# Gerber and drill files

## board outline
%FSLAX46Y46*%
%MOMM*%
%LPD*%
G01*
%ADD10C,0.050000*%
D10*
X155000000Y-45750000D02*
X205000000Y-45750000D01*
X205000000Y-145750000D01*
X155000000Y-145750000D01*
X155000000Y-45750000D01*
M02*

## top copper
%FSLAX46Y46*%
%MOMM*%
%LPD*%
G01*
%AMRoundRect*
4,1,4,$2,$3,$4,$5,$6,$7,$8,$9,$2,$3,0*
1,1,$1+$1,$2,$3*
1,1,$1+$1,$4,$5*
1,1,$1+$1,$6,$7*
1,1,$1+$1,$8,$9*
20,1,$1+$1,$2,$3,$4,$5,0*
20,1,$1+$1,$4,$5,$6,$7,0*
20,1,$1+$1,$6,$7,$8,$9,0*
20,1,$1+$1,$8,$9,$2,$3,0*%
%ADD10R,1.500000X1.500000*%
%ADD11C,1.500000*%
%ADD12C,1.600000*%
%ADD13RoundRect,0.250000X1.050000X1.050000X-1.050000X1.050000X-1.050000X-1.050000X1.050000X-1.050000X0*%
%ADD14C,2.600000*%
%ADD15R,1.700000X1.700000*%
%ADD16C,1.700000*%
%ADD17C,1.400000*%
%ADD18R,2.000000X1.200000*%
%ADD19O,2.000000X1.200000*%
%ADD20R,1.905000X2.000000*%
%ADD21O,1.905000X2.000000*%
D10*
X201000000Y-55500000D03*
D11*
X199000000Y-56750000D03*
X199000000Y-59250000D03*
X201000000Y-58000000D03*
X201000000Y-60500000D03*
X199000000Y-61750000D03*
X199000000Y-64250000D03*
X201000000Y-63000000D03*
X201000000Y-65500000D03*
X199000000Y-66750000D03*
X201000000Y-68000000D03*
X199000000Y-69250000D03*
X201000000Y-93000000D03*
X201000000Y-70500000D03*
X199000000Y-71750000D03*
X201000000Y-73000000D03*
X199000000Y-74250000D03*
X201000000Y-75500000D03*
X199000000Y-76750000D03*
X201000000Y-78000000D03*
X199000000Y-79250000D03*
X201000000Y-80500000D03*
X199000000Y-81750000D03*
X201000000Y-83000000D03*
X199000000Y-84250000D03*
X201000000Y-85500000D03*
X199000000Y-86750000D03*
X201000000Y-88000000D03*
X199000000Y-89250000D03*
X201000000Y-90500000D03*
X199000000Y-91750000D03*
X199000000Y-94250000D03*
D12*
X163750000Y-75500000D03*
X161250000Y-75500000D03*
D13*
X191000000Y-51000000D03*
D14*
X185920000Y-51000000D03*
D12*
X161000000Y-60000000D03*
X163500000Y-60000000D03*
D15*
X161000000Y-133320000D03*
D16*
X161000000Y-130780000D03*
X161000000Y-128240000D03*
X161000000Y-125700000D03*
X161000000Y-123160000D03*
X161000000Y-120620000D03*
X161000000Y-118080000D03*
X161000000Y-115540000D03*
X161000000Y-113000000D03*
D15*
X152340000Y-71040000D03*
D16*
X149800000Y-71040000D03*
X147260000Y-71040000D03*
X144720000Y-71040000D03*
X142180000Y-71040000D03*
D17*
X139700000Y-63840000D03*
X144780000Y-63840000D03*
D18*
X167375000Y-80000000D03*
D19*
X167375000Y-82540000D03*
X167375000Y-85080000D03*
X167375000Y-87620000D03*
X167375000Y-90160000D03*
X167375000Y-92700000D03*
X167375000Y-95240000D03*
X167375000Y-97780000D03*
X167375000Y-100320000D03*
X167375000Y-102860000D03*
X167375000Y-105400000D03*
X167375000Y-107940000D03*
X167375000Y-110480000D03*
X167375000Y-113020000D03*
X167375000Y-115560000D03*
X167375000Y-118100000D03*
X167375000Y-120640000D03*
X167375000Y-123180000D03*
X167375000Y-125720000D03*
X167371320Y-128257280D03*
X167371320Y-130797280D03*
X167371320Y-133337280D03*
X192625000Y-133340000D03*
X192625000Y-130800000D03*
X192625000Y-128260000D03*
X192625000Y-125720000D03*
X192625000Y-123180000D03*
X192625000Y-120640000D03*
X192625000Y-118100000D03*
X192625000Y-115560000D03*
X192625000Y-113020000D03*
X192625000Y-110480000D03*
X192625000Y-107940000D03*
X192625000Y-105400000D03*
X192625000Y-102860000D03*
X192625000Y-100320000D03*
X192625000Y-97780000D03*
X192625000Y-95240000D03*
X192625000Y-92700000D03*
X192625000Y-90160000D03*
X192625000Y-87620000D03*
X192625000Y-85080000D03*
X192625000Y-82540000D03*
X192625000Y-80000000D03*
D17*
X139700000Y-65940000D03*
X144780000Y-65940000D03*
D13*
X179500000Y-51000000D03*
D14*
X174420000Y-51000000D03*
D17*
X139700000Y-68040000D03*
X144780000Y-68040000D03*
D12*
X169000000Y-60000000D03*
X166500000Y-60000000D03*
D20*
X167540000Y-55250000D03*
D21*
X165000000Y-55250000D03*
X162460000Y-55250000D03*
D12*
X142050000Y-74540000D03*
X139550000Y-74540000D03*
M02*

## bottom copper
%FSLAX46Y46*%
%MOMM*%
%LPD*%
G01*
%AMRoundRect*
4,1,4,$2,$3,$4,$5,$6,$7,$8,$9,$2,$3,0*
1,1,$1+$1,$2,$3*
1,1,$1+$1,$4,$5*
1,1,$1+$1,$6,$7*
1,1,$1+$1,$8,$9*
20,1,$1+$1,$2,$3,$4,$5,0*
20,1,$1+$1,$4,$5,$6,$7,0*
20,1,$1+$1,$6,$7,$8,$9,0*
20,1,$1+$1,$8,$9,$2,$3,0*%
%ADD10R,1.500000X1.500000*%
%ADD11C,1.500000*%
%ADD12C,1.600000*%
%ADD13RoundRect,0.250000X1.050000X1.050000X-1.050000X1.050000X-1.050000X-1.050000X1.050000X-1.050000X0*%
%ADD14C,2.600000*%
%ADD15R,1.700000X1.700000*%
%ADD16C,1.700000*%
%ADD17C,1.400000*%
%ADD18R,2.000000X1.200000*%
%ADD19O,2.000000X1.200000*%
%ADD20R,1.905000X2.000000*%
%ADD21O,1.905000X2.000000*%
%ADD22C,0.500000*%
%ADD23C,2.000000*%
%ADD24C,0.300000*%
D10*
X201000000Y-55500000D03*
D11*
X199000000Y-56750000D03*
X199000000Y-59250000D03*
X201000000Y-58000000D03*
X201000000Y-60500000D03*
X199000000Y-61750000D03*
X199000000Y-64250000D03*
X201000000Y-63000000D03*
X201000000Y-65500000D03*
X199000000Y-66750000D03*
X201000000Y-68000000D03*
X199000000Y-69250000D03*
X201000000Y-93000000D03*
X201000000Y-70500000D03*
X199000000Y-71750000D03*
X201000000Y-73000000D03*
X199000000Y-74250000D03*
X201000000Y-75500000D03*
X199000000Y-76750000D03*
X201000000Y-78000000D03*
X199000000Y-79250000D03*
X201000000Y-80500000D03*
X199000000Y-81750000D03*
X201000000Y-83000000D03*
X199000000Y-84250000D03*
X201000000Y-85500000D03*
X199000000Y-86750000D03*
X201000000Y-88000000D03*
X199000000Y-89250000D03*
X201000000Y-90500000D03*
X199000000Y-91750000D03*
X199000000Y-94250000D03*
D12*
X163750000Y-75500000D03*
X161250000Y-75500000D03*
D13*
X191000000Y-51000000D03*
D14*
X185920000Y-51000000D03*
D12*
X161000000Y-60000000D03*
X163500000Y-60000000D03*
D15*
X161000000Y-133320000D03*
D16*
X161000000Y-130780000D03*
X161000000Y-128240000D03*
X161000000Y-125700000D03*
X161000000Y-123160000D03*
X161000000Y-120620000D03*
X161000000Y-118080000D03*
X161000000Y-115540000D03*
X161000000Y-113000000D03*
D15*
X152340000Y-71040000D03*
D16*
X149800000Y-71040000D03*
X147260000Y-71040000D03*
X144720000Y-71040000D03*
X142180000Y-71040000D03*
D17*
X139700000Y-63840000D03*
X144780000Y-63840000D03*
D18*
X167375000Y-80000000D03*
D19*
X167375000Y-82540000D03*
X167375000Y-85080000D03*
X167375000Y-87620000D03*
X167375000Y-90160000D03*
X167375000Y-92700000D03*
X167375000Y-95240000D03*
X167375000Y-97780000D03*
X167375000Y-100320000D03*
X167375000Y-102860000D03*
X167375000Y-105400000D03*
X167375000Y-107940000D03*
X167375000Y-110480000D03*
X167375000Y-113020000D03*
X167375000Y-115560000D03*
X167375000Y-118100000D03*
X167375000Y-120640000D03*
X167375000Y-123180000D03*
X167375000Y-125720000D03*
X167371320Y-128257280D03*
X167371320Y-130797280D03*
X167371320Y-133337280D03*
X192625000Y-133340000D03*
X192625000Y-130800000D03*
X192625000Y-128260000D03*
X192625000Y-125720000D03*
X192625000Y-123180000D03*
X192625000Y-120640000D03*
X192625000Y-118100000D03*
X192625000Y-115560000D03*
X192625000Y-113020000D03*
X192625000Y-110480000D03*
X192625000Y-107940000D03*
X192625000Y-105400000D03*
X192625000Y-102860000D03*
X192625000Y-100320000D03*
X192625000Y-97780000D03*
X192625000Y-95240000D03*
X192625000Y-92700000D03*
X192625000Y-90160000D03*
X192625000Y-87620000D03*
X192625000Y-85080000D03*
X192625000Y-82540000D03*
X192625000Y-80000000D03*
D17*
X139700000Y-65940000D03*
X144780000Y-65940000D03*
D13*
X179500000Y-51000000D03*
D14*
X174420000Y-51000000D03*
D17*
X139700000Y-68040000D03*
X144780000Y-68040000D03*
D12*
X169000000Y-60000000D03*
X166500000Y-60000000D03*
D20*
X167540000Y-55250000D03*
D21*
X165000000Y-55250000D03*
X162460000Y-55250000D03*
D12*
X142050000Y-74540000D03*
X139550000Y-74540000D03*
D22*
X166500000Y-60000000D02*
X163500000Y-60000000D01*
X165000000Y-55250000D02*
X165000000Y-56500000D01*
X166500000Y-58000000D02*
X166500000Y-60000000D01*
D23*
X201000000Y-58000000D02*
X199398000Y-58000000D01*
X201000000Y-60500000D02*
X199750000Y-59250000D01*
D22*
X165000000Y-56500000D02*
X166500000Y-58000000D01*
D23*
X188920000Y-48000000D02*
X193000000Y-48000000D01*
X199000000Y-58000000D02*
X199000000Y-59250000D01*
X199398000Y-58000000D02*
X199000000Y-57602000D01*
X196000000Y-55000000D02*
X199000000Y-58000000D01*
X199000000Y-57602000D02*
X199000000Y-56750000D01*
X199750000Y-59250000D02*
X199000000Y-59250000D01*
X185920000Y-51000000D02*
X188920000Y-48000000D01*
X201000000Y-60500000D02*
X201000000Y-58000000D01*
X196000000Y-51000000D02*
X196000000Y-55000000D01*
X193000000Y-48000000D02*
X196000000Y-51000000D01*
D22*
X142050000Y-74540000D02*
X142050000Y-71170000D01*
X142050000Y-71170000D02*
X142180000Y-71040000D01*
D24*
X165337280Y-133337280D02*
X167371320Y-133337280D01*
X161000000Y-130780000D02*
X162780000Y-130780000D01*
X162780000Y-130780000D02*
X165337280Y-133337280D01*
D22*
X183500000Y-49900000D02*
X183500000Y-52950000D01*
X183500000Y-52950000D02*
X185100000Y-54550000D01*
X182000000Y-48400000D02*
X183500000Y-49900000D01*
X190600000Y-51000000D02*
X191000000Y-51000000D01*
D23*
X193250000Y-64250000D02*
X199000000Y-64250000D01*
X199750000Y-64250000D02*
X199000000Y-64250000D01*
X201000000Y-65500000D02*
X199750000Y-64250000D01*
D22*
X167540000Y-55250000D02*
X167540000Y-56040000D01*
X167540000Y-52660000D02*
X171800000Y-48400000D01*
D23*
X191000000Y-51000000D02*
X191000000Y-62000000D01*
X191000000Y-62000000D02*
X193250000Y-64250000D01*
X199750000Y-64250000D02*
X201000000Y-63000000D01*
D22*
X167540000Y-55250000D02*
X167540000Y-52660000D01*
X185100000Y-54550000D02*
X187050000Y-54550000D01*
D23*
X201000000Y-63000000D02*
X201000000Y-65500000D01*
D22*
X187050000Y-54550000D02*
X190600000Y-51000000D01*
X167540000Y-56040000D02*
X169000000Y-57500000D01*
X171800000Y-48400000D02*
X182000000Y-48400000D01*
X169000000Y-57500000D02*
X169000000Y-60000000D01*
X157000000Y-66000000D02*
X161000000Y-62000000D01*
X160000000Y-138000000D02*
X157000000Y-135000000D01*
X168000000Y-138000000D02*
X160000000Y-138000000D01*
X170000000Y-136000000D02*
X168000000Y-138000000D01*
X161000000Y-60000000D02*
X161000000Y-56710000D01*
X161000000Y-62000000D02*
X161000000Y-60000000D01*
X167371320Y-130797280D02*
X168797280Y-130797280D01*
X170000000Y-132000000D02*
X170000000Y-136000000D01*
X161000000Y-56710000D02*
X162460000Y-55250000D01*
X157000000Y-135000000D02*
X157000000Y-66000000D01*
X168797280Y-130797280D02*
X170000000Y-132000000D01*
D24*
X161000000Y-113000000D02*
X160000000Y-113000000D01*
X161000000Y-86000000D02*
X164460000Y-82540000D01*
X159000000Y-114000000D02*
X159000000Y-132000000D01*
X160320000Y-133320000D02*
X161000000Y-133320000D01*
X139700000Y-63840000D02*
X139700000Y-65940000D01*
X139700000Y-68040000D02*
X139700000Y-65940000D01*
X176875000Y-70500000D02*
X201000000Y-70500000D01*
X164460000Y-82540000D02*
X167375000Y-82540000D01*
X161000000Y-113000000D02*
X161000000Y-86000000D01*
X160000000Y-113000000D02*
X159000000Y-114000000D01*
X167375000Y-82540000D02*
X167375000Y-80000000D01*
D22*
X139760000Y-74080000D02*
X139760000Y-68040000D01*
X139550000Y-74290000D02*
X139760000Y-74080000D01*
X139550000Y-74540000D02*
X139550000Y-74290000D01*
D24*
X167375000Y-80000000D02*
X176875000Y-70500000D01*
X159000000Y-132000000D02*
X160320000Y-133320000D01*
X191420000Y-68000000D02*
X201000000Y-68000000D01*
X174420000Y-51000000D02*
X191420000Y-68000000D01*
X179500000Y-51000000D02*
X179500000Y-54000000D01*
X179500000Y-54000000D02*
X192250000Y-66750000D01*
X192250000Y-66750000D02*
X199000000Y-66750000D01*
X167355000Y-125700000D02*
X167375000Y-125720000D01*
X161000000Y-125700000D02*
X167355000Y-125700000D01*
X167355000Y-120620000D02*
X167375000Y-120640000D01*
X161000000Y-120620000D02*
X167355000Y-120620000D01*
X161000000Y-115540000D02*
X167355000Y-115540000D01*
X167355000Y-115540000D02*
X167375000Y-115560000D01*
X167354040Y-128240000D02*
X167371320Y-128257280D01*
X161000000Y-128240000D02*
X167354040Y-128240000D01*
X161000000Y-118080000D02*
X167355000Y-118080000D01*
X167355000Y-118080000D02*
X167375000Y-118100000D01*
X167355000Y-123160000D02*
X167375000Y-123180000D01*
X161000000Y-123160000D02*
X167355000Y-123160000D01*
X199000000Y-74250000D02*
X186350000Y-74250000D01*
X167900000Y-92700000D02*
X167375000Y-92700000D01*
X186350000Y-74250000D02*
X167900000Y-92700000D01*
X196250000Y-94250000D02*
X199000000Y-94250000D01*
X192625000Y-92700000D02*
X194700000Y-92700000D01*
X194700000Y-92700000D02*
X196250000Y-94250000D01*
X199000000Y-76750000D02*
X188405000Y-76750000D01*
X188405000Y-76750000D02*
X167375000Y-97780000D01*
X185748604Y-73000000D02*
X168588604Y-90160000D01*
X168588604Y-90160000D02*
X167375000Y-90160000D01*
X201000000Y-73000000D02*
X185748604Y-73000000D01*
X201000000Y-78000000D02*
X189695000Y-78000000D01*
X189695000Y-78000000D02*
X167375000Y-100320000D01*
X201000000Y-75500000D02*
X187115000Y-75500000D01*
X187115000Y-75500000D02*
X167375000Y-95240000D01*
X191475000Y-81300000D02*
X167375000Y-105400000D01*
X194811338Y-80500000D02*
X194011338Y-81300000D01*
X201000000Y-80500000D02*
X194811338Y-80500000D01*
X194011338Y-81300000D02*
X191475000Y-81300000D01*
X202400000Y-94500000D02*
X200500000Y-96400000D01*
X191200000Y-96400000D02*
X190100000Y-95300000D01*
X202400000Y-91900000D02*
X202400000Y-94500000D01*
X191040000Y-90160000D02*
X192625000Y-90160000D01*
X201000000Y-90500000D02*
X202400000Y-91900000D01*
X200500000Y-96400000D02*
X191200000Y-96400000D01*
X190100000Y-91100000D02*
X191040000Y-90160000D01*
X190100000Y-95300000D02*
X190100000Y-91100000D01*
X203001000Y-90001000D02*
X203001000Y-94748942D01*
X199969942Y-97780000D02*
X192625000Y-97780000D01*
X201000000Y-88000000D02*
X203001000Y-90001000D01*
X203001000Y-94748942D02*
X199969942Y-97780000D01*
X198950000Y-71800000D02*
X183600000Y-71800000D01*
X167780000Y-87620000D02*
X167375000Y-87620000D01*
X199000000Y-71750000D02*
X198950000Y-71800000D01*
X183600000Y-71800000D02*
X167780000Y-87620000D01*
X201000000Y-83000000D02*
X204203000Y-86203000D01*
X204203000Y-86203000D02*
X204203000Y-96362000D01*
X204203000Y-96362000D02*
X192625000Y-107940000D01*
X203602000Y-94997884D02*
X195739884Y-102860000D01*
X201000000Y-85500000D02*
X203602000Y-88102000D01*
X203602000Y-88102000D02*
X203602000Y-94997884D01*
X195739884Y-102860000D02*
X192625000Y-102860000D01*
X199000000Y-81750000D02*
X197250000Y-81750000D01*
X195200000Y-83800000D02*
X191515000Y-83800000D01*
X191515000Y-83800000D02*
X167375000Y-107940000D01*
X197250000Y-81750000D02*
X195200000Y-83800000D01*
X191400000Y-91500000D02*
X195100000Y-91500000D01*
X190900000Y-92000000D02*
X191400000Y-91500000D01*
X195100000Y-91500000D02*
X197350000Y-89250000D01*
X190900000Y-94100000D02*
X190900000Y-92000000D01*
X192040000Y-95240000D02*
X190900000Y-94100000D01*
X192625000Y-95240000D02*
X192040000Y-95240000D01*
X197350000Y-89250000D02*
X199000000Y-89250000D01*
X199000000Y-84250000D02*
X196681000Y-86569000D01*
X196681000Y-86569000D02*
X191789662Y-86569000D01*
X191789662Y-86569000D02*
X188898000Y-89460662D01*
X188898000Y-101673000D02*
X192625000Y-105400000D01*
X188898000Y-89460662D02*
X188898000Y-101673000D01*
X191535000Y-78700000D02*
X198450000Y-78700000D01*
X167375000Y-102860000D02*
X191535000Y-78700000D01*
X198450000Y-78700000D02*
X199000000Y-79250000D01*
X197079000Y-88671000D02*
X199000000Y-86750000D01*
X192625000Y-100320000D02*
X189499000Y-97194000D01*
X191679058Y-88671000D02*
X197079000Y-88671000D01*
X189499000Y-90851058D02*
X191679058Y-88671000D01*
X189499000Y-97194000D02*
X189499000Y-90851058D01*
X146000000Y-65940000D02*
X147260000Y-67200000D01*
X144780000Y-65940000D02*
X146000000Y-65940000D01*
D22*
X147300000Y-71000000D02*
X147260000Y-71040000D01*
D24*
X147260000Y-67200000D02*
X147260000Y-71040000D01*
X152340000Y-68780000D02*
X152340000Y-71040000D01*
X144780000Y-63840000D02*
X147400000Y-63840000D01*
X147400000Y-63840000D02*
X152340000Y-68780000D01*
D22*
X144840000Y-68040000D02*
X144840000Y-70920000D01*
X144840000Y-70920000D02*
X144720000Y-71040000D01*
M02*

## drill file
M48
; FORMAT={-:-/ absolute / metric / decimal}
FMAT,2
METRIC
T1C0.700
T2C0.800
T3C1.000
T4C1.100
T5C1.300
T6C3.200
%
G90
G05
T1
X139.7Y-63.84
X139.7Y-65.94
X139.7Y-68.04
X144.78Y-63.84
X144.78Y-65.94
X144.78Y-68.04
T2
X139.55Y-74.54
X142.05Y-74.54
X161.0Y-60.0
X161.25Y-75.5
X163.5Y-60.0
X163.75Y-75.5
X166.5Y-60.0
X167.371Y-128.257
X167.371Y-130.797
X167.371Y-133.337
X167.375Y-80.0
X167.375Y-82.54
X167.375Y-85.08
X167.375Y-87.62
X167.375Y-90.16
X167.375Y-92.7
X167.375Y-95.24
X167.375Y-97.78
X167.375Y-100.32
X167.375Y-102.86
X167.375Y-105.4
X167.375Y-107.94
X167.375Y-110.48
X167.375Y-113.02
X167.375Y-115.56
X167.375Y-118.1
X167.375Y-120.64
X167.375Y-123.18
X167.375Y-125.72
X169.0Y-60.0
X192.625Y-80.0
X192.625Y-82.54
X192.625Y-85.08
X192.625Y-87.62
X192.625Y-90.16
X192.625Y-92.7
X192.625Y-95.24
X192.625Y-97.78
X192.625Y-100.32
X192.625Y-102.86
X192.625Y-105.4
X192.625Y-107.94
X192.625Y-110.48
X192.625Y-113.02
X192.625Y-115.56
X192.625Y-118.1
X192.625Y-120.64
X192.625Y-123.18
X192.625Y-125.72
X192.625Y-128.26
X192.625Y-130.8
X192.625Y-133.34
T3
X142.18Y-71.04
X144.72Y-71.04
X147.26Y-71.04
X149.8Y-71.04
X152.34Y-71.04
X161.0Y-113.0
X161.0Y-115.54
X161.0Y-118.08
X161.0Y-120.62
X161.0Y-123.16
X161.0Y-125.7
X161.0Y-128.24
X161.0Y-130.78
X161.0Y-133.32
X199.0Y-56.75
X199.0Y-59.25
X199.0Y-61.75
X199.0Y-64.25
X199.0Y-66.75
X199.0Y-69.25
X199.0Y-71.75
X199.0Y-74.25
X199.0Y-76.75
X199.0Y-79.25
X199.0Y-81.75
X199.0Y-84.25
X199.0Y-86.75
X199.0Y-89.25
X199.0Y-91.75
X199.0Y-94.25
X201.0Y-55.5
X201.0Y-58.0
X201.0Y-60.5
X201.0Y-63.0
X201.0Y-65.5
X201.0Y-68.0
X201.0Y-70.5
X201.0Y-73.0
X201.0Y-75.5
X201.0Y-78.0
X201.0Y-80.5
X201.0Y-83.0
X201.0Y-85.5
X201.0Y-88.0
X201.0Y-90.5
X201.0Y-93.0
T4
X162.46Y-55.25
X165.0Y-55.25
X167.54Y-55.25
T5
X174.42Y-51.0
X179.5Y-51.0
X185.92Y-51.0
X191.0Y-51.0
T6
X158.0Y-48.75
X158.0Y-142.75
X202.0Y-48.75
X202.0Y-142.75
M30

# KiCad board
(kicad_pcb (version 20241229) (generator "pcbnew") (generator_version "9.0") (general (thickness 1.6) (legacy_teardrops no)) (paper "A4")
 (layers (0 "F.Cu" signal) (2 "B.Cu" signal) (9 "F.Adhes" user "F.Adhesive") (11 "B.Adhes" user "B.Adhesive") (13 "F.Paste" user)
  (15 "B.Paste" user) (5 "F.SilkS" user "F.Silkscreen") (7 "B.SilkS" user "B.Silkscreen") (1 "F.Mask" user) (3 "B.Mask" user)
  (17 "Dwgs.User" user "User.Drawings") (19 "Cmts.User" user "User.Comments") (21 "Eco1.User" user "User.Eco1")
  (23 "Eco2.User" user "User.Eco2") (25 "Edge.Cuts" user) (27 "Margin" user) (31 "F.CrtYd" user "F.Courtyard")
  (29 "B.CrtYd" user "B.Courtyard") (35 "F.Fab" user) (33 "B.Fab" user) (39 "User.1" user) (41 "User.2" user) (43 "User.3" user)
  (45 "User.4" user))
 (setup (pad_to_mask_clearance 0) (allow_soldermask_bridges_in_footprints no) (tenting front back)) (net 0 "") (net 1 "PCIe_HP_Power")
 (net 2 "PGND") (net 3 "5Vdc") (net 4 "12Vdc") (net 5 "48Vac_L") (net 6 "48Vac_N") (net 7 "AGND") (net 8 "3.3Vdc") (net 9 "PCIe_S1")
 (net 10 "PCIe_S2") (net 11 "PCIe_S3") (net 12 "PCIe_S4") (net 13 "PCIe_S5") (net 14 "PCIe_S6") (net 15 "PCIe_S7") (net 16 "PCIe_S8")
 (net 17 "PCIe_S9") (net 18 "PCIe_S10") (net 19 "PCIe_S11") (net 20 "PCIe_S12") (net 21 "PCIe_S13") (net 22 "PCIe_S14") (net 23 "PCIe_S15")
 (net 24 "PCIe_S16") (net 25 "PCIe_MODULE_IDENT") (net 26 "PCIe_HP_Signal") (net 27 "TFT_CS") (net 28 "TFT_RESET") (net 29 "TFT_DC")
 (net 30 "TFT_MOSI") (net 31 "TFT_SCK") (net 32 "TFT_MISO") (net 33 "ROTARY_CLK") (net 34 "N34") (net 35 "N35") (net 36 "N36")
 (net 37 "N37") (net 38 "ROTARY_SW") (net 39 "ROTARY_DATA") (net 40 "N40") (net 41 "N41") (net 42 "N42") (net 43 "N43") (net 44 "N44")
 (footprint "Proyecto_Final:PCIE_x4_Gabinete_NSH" (layer "F.Cu") (at 201 55.5)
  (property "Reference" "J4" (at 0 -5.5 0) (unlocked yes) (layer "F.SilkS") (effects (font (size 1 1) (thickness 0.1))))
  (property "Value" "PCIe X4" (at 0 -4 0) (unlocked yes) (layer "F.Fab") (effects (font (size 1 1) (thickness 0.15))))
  (pad "1" thru_hole rect (at 0 0 180) (size 1.5 1.5) (drill 1) (layers "*.Cu" "*.Mask") (remove_unused_layers no) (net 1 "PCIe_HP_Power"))
  (pad "2" thru_hole circle (at -2 1.25 180) (size 1.5 1.5) (drill 1) (layers "*.Cu" "*.Mask") (remove_unused_layers no) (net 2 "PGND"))
  (pad "2" thru_hole circle (at -2 3.75 180) (size 1.5 1.5) (drill 1) (layers "*.Cu" "*.Mask") (remove_unused_layers no) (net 2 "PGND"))
  (pad "2" thru_hole circle (at 0 2.5 180) (size 1.5 1.5) (drill 1) (layers "*.Cu" "*.Mask") (remove_unused_layers no) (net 2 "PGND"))
  (pad "2" thru_hole circle (at 0 5 180) (size 1.5 1.5) (drill 1) (layers "*.Cu" "*.Mask") (remove_unused_layers no) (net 2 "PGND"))
  (pad "3" thru_hole circle (at -2 6.25 180) (size 1.5 1.5) (drill 1) (layers "*.Cu" "*.Mask") (remove_unused_layers no) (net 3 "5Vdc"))
  (pad "4" thru_hole circle (at -2 8.75 180) (size 1.5 1.5) (drill 1) (layers "*.Cu" "*.Mask") (remove_unused_layers no) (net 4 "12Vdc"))
  (pad "4" thru_hole circle (at 0 7.5 180) (size 1.5 1.5) (drill 1) (layers "*.Cu" "*.Mask") (remove_unused_layers no) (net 4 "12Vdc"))
  (pad "4" thru_hole circle (at 0 10 180) (size 1.5 1.5) (drill 1) (layers "*.Cu" "*.Mask") (remove_unused_layers no) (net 4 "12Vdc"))
  (pad "5" thru_hole circle (at -2 11.25 180) (size 1.5 1.5) (drill 1) (layers "*.Cu" "*.Mask") (remove_unused_layers no) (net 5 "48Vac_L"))
  (pad "6" thru_hole circle (at 0 12.5 180) (size 1.5 1.5) (drill 1) (layers "*.Cu" "*.Mask") (remove_unused_layers no) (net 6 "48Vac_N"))
  (pad "7" thru_hole circle (at -2 13.75 180) (size 1.5 1.5) (drill 1) (layers "*.Cu" "*.Mask") (remove_unused_layers no) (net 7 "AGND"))
  (pad "7" thru_hole circle (at 0 37.5 180) (size 1.5 1.5) (drill 1) (layers "*.Cu" "*.Mask") (remove_unused_layers no) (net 7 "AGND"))
  (pad "8" thru_hole circle (at 0 15 180) (size 1.5 1.5) (drill 1) (layers "*.Cu" "*.Mask") (remove_unused_layers no) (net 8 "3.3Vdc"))
  (pad "9" thru_hole circle (at -2 16.25 180) (size 1.5 1.5) (drill 1) (layers "*.Cu" "*.Mask") (remove_unused_layers no) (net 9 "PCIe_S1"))
  (pad "10" thru_hole circle (at 0 17.5 180) (size 1.5 1.5) (drill 1) (layers "*.Cu" "*.Mask") (remove_unused_layers no) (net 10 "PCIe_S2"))
  (pad "11" thru_hole circle (at -2 18.75 180) (size 1.5 1.5) (drill 1) (layers "*.Cu" "*.Mask") (remove_unused_layers no)
   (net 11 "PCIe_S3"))
  (pad "12" thru_hole circle (at 0 20 180) (size 1.5 1.5) (drill 1) (layers "*.Cu" "*.Mask") (remove_unused_layers no) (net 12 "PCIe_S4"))
  (pad "13" thru_hole circle (at -2 21.25 180) (size 1.5 1.5) (drill 1) (layers "*.Cu" "*.Mask") (remove_unused_layers no)
   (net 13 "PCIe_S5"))
  (pad "14" thru_hole circle (at 0 22.5 180) (size 1.5 1.5) (drill 1) (layers "*.Cu" "*.Mask") (remove_unused_layers no) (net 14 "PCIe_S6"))
  (pad "15" thru_hole circle (at -2 23.75 180) (size 1.5 1.5) (drill 1) (layers "*.Cu" "*.Mask") (remove_unused_layers no)
   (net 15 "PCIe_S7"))
  (pad "16" thru_hole circle (at 0 25 180) (size 1.5 1.5) (drill 1) (layers "*.Cu" "*.Mask") (remove_unused_layers no) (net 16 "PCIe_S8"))
  (pad "17" thru_hole circle (at -2 26.25 180) (size 1.5 1.5) (drill 1) (layers "*.Cu" "*.Mask") (remove_unused_layers no)
   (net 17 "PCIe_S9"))
  (pad "18" thru_hole circle (at 0 27.5 180) (size 1.5 1.5) (drill 1) (layers "*.Cu" "*.Mask") (remove_unused_layers no) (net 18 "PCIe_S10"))
  (pad "19" thru_hole circle (at -2 28.75 180) (size 1.5 1.5) (drill 1) (layers "*.Cu" "*.Mask") (remove_unused_layers no)
   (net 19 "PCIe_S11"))
  (pad "20" thru_hole circle (at 0 30 180) (size 1.5 1.5) (drill 1) (layers "*.Cu" "*.Mask") (remove_unused_layers no) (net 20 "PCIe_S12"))
  (pad "21" thru_hole circle (at -2 31.25 180) (size 1.5 1.5) (drill 1) (layers "*.Cu" "*.Mask") (remove_unused_layers no)
   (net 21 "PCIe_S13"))
  (pad "22" thru_hole circle (at 0 32.5 180) (size 1.5 1.5) (drill 1) (layers "*.Cu" "*.Mask") (remove_unused_layers no) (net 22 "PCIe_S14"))
  (pad "23" thru_hole circle (at -2 33.75 180) (size 1.5 1.5) (drill 1) (layers "*.Cu" "*.Mask") (remove_unused_layers no)
   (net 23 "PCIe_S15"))
  (pad "24" thru_hole circle (at 0 35 180) (size 1.5 1.5) (drill 1) (layers "*.Cu" "*.Mask") (remove_unused_layers no) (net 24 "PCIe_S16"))
  (pad "25" thru_hole circle (at -2 36.25 180) (size 1.5 1.5) (drill 1) (layers "*.Cu" "*.Mask") (remove_unused_layers no)
   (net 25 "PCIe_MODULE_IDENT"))
  (pad "26" thru_hole circle (at -2 38.75 180) (size 1.5 1.5) (drill 1) (layers "*.Cu" "*.Mask") (remove_unused_layers no)
   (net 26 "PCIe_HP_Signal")))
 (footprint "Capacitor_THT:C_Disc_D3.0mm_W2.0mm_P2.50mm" (layer "F.Cu") (at 163.75 75.5 180)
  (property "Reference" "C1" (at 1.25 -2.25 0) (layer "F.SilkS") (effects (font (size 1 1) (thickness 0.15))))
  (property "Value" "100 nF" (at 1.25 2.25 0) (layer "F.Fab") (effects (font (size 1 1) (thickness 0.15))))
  (pad "1" thru_hole circle (at 0 0 180) (size 1.6 1.6) (drill 0.8) (layers "*.Cu" "*.Mask") (remove_unused_layers no) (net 2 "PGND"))
  (pad "2" thru_hole circle (at 2.5 0 180) (size 1.6 1.6) (drill 0.8) (layers "*.Cu" "*.Mask") (remove_unused_layers no) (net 7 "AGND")))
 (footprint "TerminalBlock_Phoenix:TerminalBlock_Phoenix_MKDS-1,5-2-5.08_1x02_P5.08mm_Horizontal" (layer "F.Cu") (at 191 51 180)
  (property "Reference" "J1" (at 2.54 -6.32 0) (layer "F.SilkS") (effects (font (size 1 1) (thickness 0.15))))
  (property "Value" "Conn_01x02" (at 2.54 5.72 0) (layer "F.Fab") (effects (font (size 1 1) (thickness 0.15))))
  (pad "1" thru_hole roundrect (at 0 0 180) (size 2.6 2.6) (drill 1.3) (layers "*.Cu" "*.Mask") (remove_unused_layers no)
   (roundrect_rratio 0.096154) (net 4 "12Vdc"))
  (pad "2" thru_hole circle (at 5.08 0 180) (size 2.6 2.6) (drill 1.3) (layers "*.Cu" "*.Mask") (remove_unused_layers no) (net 2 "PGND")))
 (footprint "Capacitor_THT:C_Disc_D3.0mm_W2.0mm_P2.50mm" (layer "F.Cu") (at 161 60)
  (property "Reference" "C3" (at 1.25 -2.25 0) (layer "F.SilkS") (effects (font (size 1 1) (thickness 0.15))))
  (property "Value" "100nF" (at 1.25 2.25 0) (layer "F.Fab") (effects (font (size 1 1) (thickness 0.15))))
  (pad "1" thru_hole circle (at 0 0) (size 1.6 1.6) (drill 0.8) (layers "*.Cu" "*.Mask") (remove_unused_layers no) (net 3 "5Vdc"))
  (pad "2" thru_hole circle (at 2.5 0) (size 1.6 1.6) (drill 0.8) (layers "*.Cu" "*.Mask") (remove_unused_layers no) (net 2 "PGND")))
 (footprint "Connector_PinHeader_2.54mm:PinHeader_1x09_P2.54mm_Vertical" (layer "F.Cu") (at 161 133.32 180)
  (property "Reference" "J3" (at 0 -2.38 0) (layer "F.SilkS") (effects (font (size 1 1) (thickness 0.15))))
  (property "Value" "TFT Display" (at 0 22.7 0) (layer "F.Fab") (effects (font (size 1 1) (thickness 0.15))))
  (pad "1" thru_hole rect (at 0 0 180) (size 1.7 1.7) (drill 1) (layers "*.Cu" "*.Mask") (remove_unused_layers no) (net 8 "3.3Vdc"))
  (pad "2" thru_hole circle (at 0 2.54 180) (size 1.7 1.7) (drill 1) (layers "*.Cu" "*.Mask") (remove_unused_layers no) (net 7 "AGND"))
  (pad "3" thru_hole circle (at 0 5.08 180) (size 1.7 1.7) (drill 1) (layers "*.Cu" "*.Mask") (remove_unused_layers no) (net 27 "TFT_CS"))
  (pad "4" thru_hole circle (at 0 7.62 180) (size 1.7 1.7) (drill 1) (layers "*.Cu" "*.Mask") (remove_unused_layers no) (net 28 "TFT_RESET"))
  (pad "5" thru_hole circle (at 0 10.16 180) (size 1.7 1.7) (drill 1) (layers "*.Cu" "*.Mask") (remove_unused_layers no) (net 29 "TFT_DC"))
  (pad "6" thru_hole circle (at 0 12.7 180) (size 1.7 1.7) (drill 1) (layers "*.Cu" "*.Mask") (remove_unused_layers no) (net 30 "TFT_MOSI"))
  (pad "7" thru_hole circle (at 0 15.24 180) (size 1.7 1.7) (drill 1) (layers "*.Cu" "*.Mask") (remove_unused_layers no) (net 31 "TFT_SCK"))
  (pad "8" thru_hole circle (at 0 17.78 180) (size 1.7 1.7) (drill 1) (layers "*.Cu" "*.Mask") (remove_unused_layers no) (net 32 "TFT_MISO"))
  (pad "9" thru_hole circle (at 0 20.32 180) (size 1.7 1.7) (drill 1) (layers "*.Cu" "*.Mask") (remove_unused_layers no) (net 8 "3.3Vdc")))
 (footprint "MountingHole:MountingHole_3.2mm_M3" (layer "F.Cu") (at 202 142.75)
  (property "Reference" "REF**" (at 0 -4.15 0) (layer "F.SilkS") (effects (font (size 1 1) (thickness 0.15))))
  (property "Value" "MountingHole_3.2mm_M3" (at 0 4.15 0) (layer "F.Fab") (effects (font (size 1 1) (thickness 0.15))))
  (pad "" np_thru_hole circle (at 0 0) (size 3.2 3.2) (drill 3.2) (layers "*.Cu" "*.Mask")))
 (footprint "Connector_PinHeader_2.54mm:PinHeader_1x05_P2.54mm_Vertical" (layer "F.Cu") (at 152.34 71.04 -90)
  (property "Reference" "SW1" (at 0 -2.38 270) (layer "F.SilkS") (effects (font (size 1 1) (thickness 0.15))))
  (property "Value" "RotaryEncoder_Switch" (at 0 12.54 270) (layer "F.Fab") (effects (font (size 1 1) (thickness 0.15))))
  (pad "1" thru_hole rect (at 0 0 270) (size 1.7 1.7) (drill 1) (layers "*.Cu" "*.Mask") (remove_unused_layers no))
  (pad "2" thru_hole circle (at 0 2.54 270) (size 1.7 1.7) (drill 1) (layers "*.Cu" "*.Mask") (remove_unused_layers no))
  (pad "3" thru_hole circle (at 0 5.08 270) (size 1.7 1.7) (drill 1) (layers "*.Cu" "*.Mask") (remove_unused_layers no))
  (pad "4" thru_hole circle (at 0 7.62 270) (size 1.7 1.7) (drill 1) (layers "*.Cu" "*.Mask") (remove_unused_layers no))
  (pad "5" thru_hole circle (at 0 10.16 270) (size 1.7 1.7) (drill 1) (layers "*.Cu" "*.Mask") (remove_unused_layers no)))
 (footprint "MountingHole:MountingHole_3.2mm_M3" (layer "F.Cu") (at 158 48.75)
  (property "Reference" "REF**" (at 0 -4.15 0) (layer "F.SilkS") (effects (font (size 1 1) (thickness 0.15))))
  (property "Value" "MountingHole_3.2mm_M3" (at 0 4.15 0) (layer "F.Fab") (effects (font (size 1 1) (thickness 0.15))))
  (pad "" np_thru_hole circle (at 0 0) (size 3.2 3.2) (drill 3.2) (layers "*.Cu" "*.Mask")))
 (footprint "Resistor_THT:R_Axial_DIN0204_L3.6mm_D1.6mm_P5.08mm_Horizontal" (layer "F.Cu") (at 139.7 63.84)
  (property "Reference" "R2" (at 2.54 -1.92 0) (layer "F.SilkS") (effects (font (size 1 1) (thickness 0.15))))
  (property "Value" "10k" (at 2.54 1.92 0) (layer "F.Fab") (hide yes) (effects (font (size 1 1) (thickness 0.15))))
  (pad "1" thru_hole circle (at 0 0) (size 1.4 1.4) (drill 0.7) (layers "*.Cu" "*.Mask") (remove_unused_layers no) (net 8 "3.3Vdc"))
  (pad "2" thru_hole circle (at 5.08 0) (size 1.4 1.4) (drill 0.7) (layers "*.Cu" "*.Mask") (remove_unused_layers no) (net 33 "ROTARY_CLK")))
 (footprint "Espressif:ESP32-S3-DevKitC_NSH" (layer "F.Cu") (at 167.375 80)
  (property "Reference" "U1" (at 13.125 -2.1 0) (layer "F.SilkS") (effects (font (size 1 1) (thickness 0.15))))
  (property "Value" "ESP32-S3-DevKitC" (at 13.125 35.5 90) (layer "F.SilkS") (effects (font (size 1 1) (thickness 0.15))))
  (pad "1" thru_hole rect (at 0 0 270) (size 1.2 2) (drill 0.8) (layers "*.Cu" "*.Mask") (remove_unused_layers no) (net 8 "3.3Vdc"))
  (pad "2" thru_hole oval (at 0 2.54 270) (size 1.2 2) (drill 0.8) (layers "*.Cu" "*.Mask") (remove_unused_layers no) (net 8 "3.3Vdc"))
  (pad "3" thru_hole oval (at 0 5.08 270) (size 1.2 2) (drill 0.8) (layers "*.Cu" "*.Mask") (remove_unused_layers no) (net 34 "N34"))
  (pad "4" thru_hole oval (at 0 7.62 270) (size 1.2 2) (drill 0.8) (layers "*.Cu" "*.Mask") (remove_unused_layers no) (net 9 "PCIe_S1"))
  (pad "5" thru_hole oval (at 0 10.16 270) (size 1.2 2) (drill 0.8) (layers "*.Cu" "*.Mask") (remove_unused_layers no) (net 10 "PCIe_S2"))
  (pad "6" thru_hole oval (at 0 12.7 270) (size 1.2 2) (drill 0.8) (layers "*.Cu" "*.Mask") (remove_unused_layers no) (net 11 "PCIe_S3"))
  (pad "7" thru_hole oval (at 0 15.24 270) (size 1.2 2) (drill 0.8) (layers "*.Cu" "*.Mask") (remove_unused_layers no) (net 12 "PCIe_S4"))
  (pad "8" thru_hole oval (at 0 17.78 270) (size 1.2 2) (drill 0.8) (layers "*.Cu" "*.Mask") (remove_unused_layers no) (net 13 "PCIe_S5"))
  (pad "9" thru_hole oval (at 0 20.32 270) (size 1.2 2) (drill 0.8) (layers "*.Cu" "*.Mask") (remove_unused_layers no) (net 14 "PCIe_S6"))
  (pad "10" thru_hole oval (at 0 22.86 270) (size 1.2 2) (drill 0.8) (layers "*.Cu" "*.Mask") (remove_unused_layers no) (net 15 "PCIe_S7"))
  (pad "11" thru_hole oval (at 0 25.4 270) (size 1.2 2) (drill 0.8) (layers "*.Cu" "*.Mask") (remove_unused_layers no) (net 16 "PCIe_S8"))
  (pad "12" thru_hole oval (at 0 27.94 270) (size 1.2 2) (drill 0.8) (layers "*.Cu" "*.Mask") (remove_unused_layers no) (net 17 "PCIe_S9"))
  (pad "13" thru_hole oval (at 0 30.48 270) (size 1.2 2) (drill 0.8) (layers "*.Cu" "*.Mask") (remove_unused_layers no)
   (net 25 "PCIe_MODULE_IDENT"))
  (pad "14" thru_hole oval (at 0 33.02 270) (size 1.2 2) (drill 0.8) (layers "*.Cu" "*.Mask") (remove_unused_layers no) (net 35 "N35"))
  (pad "15" thru_hole oval (at 0 35.56 270) (size 1.2 2) (drill 0.8) (layers "*.Cu" "*.Mask") (remove_unused_layers no) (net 32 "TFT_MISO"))
  (pad "16" thru_hole oval (at 0 38.1 270) (size 1.2 2) (drill 0.8) (layers "*.Cu" "*.Mask") (remove_unused_layers no) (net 31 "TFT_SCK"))
  (pad "17" thru_hole oval (at 0 40.64 270) (size 1.2 2) (drill 0.8) (layers "*.Cu" "*.Mask") (remove_unused_layers no) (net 30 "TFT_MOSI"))
  (pad "18" thru_hole oval (at 0 43.18 270) (size 1.2 2) (drill 0.8) (layers "*.Cu" "*.Mask") (remove_unused_layers no) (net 29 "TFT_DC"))
  (pad "19" thru_hole oval (at 0 45.72 270) (size 1.2 2) (drill 0.8) (layers "*.Cu" "*.Mask") (remove_unused_layers no) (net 28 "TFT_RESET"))
  (pad "20" thru_hole oval (at -0.00368 48.25728 270) (size 1.2 2) (drill 0.8) (layers "*.Cu" "*.Mask") (remove_unused_layers no)
   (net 27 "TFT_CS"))
  (pad "21" thru_hole oval (at -0.00368 50.79728 270) (size 1.2 2) (drill 0.8) (layers "*.Cu" "*.Mask") (remove_unused_layers no)
   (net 3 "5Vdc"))
  (pad "22" thru_hole oval (at -0.00368 53.33728 270) (size 1.2 2) (drill 0.8) (layers "*.Cu" "*.Mask") (remove_unused_layers no)
   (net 7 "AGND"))
  (pad "23" thru_hole oval (at 25.25 53.34 270) (size 1.2 2) (drill 0.8) (layers "*.Cu" "*.Mask") (remove_unused_layers no) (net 7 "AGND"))
  (pad "24" thru_hole oval (at 25.25 50.8 270) (size 1.2 2) (drill 0.8) (layers "*.Cu" "*.Mask") (remove_unused_layers no) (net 7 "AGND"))
  (pad "25" thru_hole oval (at 25.25 48.26 270) (size 1.2 2) (drill 0.8) (layers "*.Cu" "*.Mask") (remove_unused_layers no) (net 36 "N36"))
  (pad "26" thru_hole oval (at 25.25 45.72 270) (size 1.2 2) (drill 0.8) (layers "*.Cu" "*.Mask") (remove_unused_layers no) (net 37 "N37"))
  (pad "27" thru_hole oval (at 25.25 43.18 270) (size 1.2 2) (drill 0.8) (layers "*.Cu" "*.Mask") (remove_unused_layers no)
   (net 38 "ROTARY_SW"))
  (pad "28" thru_hole oval (at 25.25 40.64 270) (size 1.2 2) (drill 0.8) (layers "*.Cu" "*.Mask") (remove_unused_layers no)
   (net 33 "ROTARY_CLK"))
  (pad "29" thru_hole oval (at 25.25 38.1 270) (size 1.2 2) (drill 0.8) (layers "*.Cu" "*.Mask") (remove_unused_layers no)
   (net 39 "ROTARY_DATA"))
  (pad "30" thru_hole oval (at 25.25 35.56 270) (size 1.2 2) (drill 0.8) (layers "*.Cu" "*.Mask") (remove_unused_layers no) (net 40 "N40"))
  (pad "31" thru_hole oval (at 25.25 33.02 270) (size 1.2 2) (drill 0.8) (layers "*.Cu" "*.Mask") (remove_unused_layers no) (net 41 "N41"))
  (pad "32" thru_hole oval (at 25.25 30.48 270) (size 1.2 2) (drill 0.8) (layers "*.Cu" "*.Mask") (remove_unused_layers no)
   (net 1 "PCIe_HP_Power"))
  (pad "33" thru_hole oval (at 25.25 27.94 270) (size 1.2 2) (drill 0.8) (layers "*.Cu" "*.Mask") (remove_unused_layers no)
   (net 18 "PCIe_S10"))
  (pad "34" thru_hole oval (at 25.25 25.4 270) (size 1.2 2) (drill 0.8) (layers "*.Cu" "*.Mask") (remove_unused_layers no)
   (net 19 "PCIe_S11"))
  (pad "35" thru_hole oval (at 25.25 22.86 270) (size 1.2 2) (drill 0.8) (layers "*.Cu" "*.Mask") (remove_unused_layers no)
   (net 20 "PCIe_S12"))
  (pad "36" thru_hole oval (at 25.25 20.32 270) (size 1.2 2) (drill 0.8) (layers "*.Cu" "*.Mask") (remove_unused_layers no)
   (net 21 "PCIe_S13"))
  (pad "37" thru_hole oval (at 25.25 17.78 270) (size 1.2 2) (drill 0.8) (layers "*.Cu" "*.Mask") (remove_unused_layers no)
   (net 22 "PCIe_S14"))
  (pad "38" thru_hole oval (at 25.25 15.24 270) (size 1.2 2) (drill 0.8) (layers "*.Cu" "*.Mask") (remove_unused_layers no)
   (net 23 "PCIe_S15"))
  (pad "39" thru_hole oval (at 25.25 12.7 270) (size 1.2 2) (drill 0.8) (layers "*.Cu" "*.Mask") (remove_unused_layers no)
   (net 26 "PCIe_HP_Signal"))
  (pad "40" thru_hole oval (at 25.25 10.16 270) (size 1.2 2) (drill 0.8) (layers "*.Cu" "*.Mask") (remove_unused_layers no)
   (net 24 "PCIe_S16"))
  (pad "41" thru_hole oval (at 25.25 7.62 270) (size 1.2 2) (drill 0.8) (layers "*.Cu" "*.Mask") (remove_unused_layers no) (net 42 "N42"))
  (pad "42" thru_hole oval (at 25.25 5.08 270) (size 1.2 2) (drill 0.8) (layers "*.Cu" "*.Mask") (remove_unused_layers no) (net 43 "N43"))
  (pad "43" thru_hole oval (at 25.25 2.54 270) (size 1.2 2) (drill 0.8) (layers "*.Cu" "*.Mask") (remove_unused_layers no) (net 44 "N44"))
  (pad "44" thru_hole oval (at 25.25 0 270) (size 1.2 2) (drill 0.8) (layers "*.Cu" "*.Mask") (remove_unused_layers no) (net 7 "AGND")))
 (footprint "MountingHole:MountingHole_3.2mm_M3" (layer "F.Cu") (at 158 142.75)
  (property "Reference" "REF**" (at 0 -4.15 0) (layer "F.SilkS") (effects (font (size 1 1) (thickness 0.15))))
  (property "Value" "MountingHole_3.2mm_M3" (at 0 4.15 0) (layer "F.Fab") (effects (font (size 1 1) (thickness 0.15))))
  (pad "" np_thru_hole circle (at 0 0) (size 3.2 3.2) (drill 3.2) (layers "*.Cu" "*.Mask")))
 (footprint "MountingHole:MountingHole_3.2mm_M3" (layer "F.Cu") (at 202 48.75)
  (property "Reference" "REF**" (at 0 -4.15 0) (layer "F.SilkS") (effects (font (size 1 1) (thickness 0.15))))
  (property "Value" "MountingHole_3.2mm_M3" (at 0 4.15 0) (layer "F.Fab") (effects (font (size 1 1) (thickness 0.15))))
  (pad "" np_thru_hole circle (at 0 0) (size 3.2 3.2) (drill 3.2) (layers "*.Cu" "*.Mask")))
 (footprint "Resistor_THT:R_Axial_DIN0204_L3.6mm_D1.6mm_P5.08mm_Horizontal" (layer "F.Cu") (at 139.7 65.94)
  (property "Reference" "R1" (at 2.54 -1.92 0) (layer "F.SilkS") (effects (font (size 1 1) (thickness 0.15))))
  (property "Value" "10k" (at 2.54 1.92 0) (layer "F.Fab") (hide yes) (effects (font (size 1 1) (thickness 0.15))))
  (pad "1" thru_hole circle (at 0 0) (size 1.4 1.4) (drill 0.7) (layers "*.Cu" "*.Mask") (remove_unused_layers no) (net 8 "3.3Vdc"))
  (pad "2" thru_hole circle (at 5.08 0) (size 1.4 1.4) (drill 0.7) (layers "*.Cu" "*.Mask") (remove_unused_layers no) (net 39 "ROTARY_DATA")))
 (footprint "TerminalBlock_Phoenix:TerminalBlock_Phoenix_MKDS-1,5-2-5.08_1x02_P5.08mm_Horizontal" (layer "F.Cu") (at 179.5 51 180)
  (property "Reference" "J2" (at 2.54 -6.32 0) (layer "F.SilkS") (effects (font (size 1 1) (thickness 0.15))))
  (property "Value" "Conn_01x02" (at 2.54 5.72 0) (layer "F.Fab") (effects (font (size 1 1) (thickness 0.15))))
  (pad "1" thru_hole roundrect (at 0 0 180) (size 2.6 2.6) (drill 1.3) (layers "*.Cu" "*.Mask") (remove_unused_layers no)
   (roundrect_rratio 0.096154) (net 5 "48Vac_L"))
  (pad "2" thru_hole circle (at 5.08 0 180) (size 2.6 2.6) (drill 1.3) (layers "*.Cu" "*.Mask") (remove_unused_layers no) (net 6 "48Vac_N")))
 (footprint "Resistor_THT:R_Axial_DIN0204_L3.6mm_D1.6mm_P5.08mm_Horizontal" (layer "F.Cu") (at 139.7 68.04)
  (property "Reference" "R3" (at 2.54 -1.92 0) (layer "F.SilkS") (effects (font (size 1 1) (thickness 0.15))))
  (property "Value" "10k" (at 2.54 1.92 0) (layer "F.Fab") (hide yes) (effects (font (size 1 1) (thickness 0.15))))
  (pad "1" thru_hole circle (at 0 0) (size 1.4 1.4) (drill 0.7) (layers "*.Cu" "*.Mask") (remove_unused_layers no) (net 8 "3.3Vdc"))
  (pad "2" thru_hole circle (at 5.08 0) (size 1.4 1.4) (drill 0.7) (layers "*.Cu" "*.Mask") (remove_unused_layers no) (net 38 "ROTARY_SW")))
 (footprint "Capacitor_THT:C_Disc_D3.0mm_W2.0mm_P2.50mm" (layer "F.Cu") (at 169 60 180)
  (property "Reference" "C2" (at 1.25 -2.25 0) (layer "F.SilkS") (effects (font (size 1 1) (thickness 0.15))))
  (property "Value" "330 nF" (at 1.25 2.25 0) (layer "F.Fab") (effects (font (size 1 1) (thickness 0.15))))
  (pad "1" thru_hole circle (at 0 0 180) (size 1.6 1.6) (drill 0.8) (layers "*.Cu" "*.Mask") (remove_unused_layers no) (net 4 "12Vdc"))
  (pad "2" thru_hole circle (at 2.5 0 180) (size 1.6 1.6) (drill 0.8) (layers "*.Cu" "*.Mask") (remove_unused_layers no) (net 2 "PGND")))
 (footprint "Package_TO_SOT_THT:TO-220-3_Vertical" (layer "F.Cu") (at 167.54 55.25 180)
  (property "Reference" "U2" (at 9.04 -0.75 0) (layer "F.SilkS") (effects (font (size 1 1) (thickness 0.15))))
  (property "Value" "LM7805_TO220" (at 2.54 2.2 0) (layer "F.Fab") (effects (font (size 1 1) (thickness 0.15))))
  (pad "1" thru_hole rect (at 0 0 180) (size 1.905 2) (drill 1.1) (layers "*.Cu" "*.Mask") (remove_unused_layers no) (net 4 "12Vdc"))
  (pad "2" thru_hole oval (at 2.54 0 180) (size 1.905 2) (drill 1.1) (layers "*.Cu" "*.Mask") (remove_unused_layers no) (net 2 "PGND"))
  (pad "3" thru_hole oval (at 5.08 0 180) (size 1.905 2) (drill 1.1) (layers "*.Cu" "*.Mask") (remove_unused_layers no) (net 3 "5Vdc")))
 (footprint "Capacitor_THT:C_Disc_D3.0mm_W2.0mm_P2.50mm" (layer "F.Cu") (at 142.05 74.54 180)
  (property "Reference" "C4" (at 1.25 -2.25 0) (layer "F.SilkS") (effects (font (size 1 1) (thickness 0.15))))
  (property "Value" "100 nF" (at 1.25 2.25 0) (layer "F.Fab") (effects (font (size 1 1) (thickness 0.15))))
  (pad "1" thru_hole circle (at 0 0 180) (size 1.6 1.6) (drill 0.8) (layers "*.Cu" "*.Mask") (remove_unused_layers no) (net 7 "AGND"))
  (pad "2" thru_hole circle (at 2.5 0 180) (size 1.6 1.6) (drill 0.8) (layers "*.Cu" "*.Mask") (remove_unused_layers no) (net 8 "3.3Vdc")))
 (gr_rect (start 155 45.75) (end 205 145.75) (stroke (width 0.05) (type solid)) (fill no) (layer "Edge.Cuts"))
 (segment (start 166.5 60) (end 163.5 60) (width 0.5) (layer "B.Cu") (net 2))
 (segment (start 165 55.25) (end 165 56.5) (width 0.5) (layer "B.Cu") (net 2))
 (segment (start 166.5 58) (end 166.5 60) (width 0.5) (layer "B.Cu") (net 2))
 (segment (start 201 58) (end 199.398 58) (width 2) (layer "B.Cu") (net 2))
 (segment (start 201 60.5) (end 199.75 59.25) (width 2) (layer "B.Cu") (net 2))
 (segment (start 165 56.5) (end 166.5 58) (width 0.5) (layer "B.Cu") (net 2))
 (segment (start 188.92 48) (end 193 48) (width 2) (layer "B.Cu") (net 2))
 (segment (start 199 58) (end 199 59.25) (width 2) (layer "B.Cu") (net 2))
 (segment (start 199.398 58) (end 199 57.602) (width 2) (layer "B.Cu") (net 2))
 (segment (start 196 55) (end 199 58) (width 2) (layer "B.Cu") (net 2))
 (segment (start 199 57.602) (end 199 56.75) (width 2) (layer "B.Cu") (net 2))
 (segment (start 199.75 59.25) (end 199 59.25) (width 2) (layer "B.Cu") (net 2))
 (segment (start 185.92 51) (end 188.92 48) (width 2) (layer "B.Cu") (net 2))
 (segment (start 201 60.5) (end 201 58) (width 2) (layer "B.Cu") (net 2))
 (segment (start 196 51) (end 196 55) (width 2) (layer "B.Cu") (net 2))
 (segment (start 193 48) (end 196 51) (width 2) (layer "B.Cu") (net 2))
 (segment (start 142.05 74.54) (end 142.05 71.17) (width 0.5) (layer "B.Cu") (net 7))
 (segment (start 142.05 71.17) (end 142.18 71.04) (width 0.5) (layer "B.Cu") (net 7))
 (segment (start 165.33728 133.33728) (end 167.37132 133.33728) (width 0.3) (layer "B.Cu") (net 7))
 (segment (start 161 130.78) (end 162.78 130.78) (width 0.3) (layer "B.Cu") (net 7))
 (segment (start 162.78 130.78) (end 165.33728 133.33728) (width 0.3) (layer "B.Cu") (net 7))
 (segment (start 183.5 49.9) (end 183.5 52.95) (width 0.5) (layer "B.Cu") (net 4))
 (segment (start 183.5 52.95) (end 185.1 54.55) (width 0.5) (layer "B.Cu") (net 4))
 (segment (start 182 48.4) (end 183.5 49.9) (width 0.5) (layer "B.Cu") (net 4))
 (segment (start 190.6 51) (end 191 51) (width 0.5) (layer "B.Cu") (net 4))
 (segment (start 193.25 64.25) (end 199 64.25) (width 2) (layer "B.Cu") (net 4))
 (segment (start 199.75 64.25) (end 199 64.25) (width 2) (layer "B.Cu") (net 4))
 (segment (start 201 65.5) (end 199.75 64.25) (width 2) (layer "B.Cu") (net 4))
 (segment (start 167.54 55.25) (end 167.54 56.04) (width 0.5) (layer "B.Cu") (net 4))
 (segment (start 167.54 52.66) (end 171.8 48.4) (width 0.5) (layer "B.Cu") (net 4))
 (segment (start 191 51) (end 191 62) (width 2) (layer "B.Cu") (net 4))
 (segment (start 191 62) (end 193.25 64.25) (width 2) (layer "B.Cu") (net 4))
 (segment (start 199.75 64.25) (end 201 63) (width 2) (layer "B.Cu") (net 4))
 (segment (start 167.54 55.25) (end 167.54 52.66) (width 0.5) (layer "B.Cu") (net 4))
 (segment (start 185.1 54.55) (end 187.05 54.55) (width 0.5) (layer "B.Cu") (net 4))
 (segment (start 201 63) (end 201 65.5) (width 2) (layer "B.Cu") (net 4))
 (segment (start 187.05 54.55) (end 190.6 51) (width 0.5) (layer "B.Cu") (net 4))
 (segment (start 167.54 56.04) (end 169 57.5) (width 0.5) (layer "B.Cu") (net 4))
 (segment (start 171.8 48.4) (end 182 48.4) (width 0.5) (layer "B.Cu") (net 4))
 (segment (start 169 57.5) (end 169 60) (width 0.5) (layer "B.Cu") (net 4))
 (segment (start 157 66) (end 161 62) (width 0.5) (layer "B.Cu") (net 3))
 (segment (start 160 138) (end 157 135) (width 0.5) (layer "B.Cu") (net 3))
 (segment (start 168 138) (end 160 138) (width 0.5) (layer "B.Cu") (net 3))
 (segment (start 170 136) (end 168 138) (width 0.5) (layer "B.Cu") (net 3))
 (segment (start 161 60) (end 161 56.71) (width 0.5) (layer "B.Cu") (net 3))
 (segment (start 161 62) (end 161 60) (width 0.5) (layer "B.Cu") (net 3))
 (segment (start 167.37132 130.79728) (end 168.79728 130.79728) (width 0.5) (layer "B.Cu") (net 3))
 (segment (start 170 132) (end 170 136) (width 0.5) (layer "B.Cu") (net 3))
 (segment (start 161 56.71) (end 162.46 55.25) (width 0.5) (layer "B.Cu") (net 3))
 (segment (start 157 135) (end 157 66) (width 0.5) (layer "B.Cu") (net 3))
 (segment (start 168.79728 130.79728) (end 170 132) (width 0.5) (layer "B.Cu") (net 3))
 (segment (start 161 113) (end 160 113) (width 0.3) (layer "B.Cu") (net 8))
 (segment (start 161 86) (end 164.46 82.54) (width 0.3) (layer "B.Cu") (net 8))
 (segment (start 159 114) (end 159 132) (width 0.3) (layer "B.Cu") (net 8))
 (segment (start 160.32 133.32) (end 161 133.32) (width 0.3) (layer "B.Cu") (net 8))
 (segment (start 139.7 63.84) (end 139.7 65.94) (width 0.3) (layer "B.Cu") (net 8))
 (segment (start 139.7 68.04) (end 139.7 65.94) (width 0.3) (layer "B.Cu") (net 8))
 (segment (start 176.875 70.5) (end 201 70.5) (width 0.3) (layer "B.Cu") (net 8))
 (segment (start 164.46 82.54) (end 167.375 82.54) (width 0.3) (layer "B.Cu") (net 8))
 (segment (start 161 113) (end 161 86) (width 0.3) (layer "B.Cu") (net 8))
 (segment (start 160 113) (end 159 114) (width 0.3) (layer "B.Cu") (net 8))
 (segment (start 167.375 82.54) (end 167.375 80) (width 0.3) (layer "B.Cu") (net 8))
 (segment (start 139.76 74.08) (end 139.76 68.04) (width 0.5) (layer "B.Cu") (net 8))
 (segment (start 139.55 74.29) (end 139.76 74.08) (width 0.5) (layer "B.Cu") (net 8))
 (segment (start 139.55 74.54) (end 139.55 74.29) (width 0.5) (layer "B.Cu") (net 8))
 (segment (start 167.375 80) (end 176.875 70.5) (width 0.3) (layer "B.Cu") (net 8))
 (segment (start 159 132) (end 160.32 133.32) (width 0.3) (layer "B.Cu") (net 8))
 (segment (start 191.42 68) (end 201 68) (width 0.3) (layer "B.Cu") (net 6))
 (segment (start 174.42 51) (end 191.42 68) (width 0.3) (layer "B.Cu") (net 6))
 (segment (start 179.5 51) (end 179.5 54) (width 0.3) (layer "B.Cu") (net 5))
 (segment (start 179.5 54) (end 192.25 66.75) (width 0.3) (layer "B.Cu") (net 5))
 (segment (start 192.25 66.75) (end 199 66.75) (width 0.3) (layer "B.Cu") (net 5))
 (segment (start 167.355 125.7) (end 167.375 125.72) (width 0.3) (layer "B.Cu") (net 28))
 (segment (start 161 125.7) (end 167.355 125.7) (width 0.3) (layer "B.Cu") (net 28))
 (segment (start 167.355 120.62) (end 167.375 120.64) (width 0.3) (layer "B.Cu") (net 30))
 (segment (start 161 120.62) (end 167.355 120.62) (width 0.3) (layer "B.Cu") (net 30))
 (segment (start 161 115.54) (end 167.355 115.54) (width 0.3) (layer "B.Cu") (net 32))
 (segment (start 167.355 115.54) (end 167.375 115.56) (width 0.3) (layer "B.Cu") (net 32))
 (segment (start 167.35404 128.24) (end 167.37132 128.25728) (width 0.3) (layer "B.Cu") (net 27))
 (segment (start 161 128.24) (end 167.35404 128.24) (width 0.3) (layer "B.Cu") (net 27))
 (segment (start 161 118.08) (end 167.355 118.08) (width 0.3) (layer "B.Cu") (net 31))
 (segment (start 167.355 118.08) (end 167.375 118.1) (width 0.3) (layer "B.Cu") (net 31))
 (segment (start 167.355 123.16) (end 167.375 123.18) (width 0.3) (layer "B.Cu") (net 29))
 (segment (start 161 123.16) (end 167.355 123.16) (width 0.3) (layer "B.Cu") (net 29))
 (segment (start 199 74.25) (end 186.35 74.25) (width 0.3) (layer "B.Cu") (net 11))
 (segment (start 167.9 92.7) (end 167.375 92.7) (width 0.3) (layer "B.Cu") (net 11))
 (segment (start 186.35 74.25) (end 167.9 92.7) (width 0.3) (layer "B.Cu") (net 11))
 (segment (start 196.25 94.25) (end 199 94.25) (width 0.3) (layer "B.Cu") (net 26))
 (segment (start 192.625 92.7) (end 194.7 92.7) (width 0.3) (layer "B.Cu") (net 26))
 (segment (start 194.7 92.7) (end 196.25 94.25) (width 0.3) (layer "B.Cu") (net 26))
 (segment (start 199 76.75) (end 188.405 76.75) (width 0.3) (layer "B.Cu") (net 13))
 (segment (start 188.405 76.75) (end 167.375 97.78) (width 0.3) (layer "B.Cu") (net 13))
 (segment (start 185.748604 73) (end 168.588604 90.16) (width 0.3) (layer "B.Cu") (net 10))
 (segment (start 168.588604 90.16) (end 167.375 90.16) (width 0.3) (layer "B.Cu") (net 10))
 (segment (start 201 73) (end 185.748604 73) (width 0.3) (layer "B.Cu") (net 10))
 (segment (start 201 78) (end 189.695 78) (width 0.3) (layer "B.Cu") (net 14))
 (segment (start 189.695 78) (end 167.375 100.32) (width 0.3) (layer "B.Cu") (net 14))
 (segment (start 201 75.5) (end 187.115 75.5) (width 0.3) (layer "B.Cu") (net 12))
 (segment (start 187.115 75.5) (end 167.375 95.24) (width 0.3) (layer "B.Cu") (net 12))
 (segment (start 191.475 81.3) (end 167.375 105.4) (width 0.3) (layer "B.Cu") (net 16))
 (segment (start 194.811338 80.5) (end 194.011338 81.3) (width 0.3) (layer "B.Cu") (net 16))
 (segment (start 201 80.5) (end 194.811338 80.5) (width 0.3) (layer "B.Cu") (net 16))
 (segment (start 194.011338 81.3) (end 191.475 81.3) (width 0.3) (layer "B.Cu") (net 16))
 (segment (start 202.4 94.5) (end 200.5 96.4) (width 0.3) (layer "B.Cu") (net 24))
 (segment (start 191.2 96.4) (end 190.1 95.3) (width 0.3) (layer "B.Cu") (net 24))
 (segment (start 202.4 91.9) (end 202.4 94.5) (width 0.3) (layer "B.Cu") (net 24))
 (segment (start 191.04 90.16) (end 192.625 90.16) (width 0.3) (layer "B.Cu") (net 24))
 (segment (start 201 90.5) (end 202.4 91.9) (width 0.3) (layer "B.Cu") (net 24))
 (segment (start 200.5 96.4) (end 191.2 96.4) (width 0.3) (layer "B.Cu") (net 24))
 (segment (start 190.1 91.1) (end 191.04 90.16) (width 0.3) (layer "B.Cu") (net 24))
 (segment (start 190.1 95.3) (end 190.1 91.1) (width 0.3) (layer "B.Cu") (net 24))
 (segment (start 203.001 90.001) (end 203.001 94.748942) (width 0.3) (layer "B.Cu") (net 22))
 (segment (start 199.969942 97.78) (end 192.625 97.78) (width 0.3) (layer "B.Cu") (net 22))
 (segment (start 201 88) (end 203.001 90.001) (width 0.3) (layer "B.Cu") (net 22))
 (segment (start 203.001 94.748942) (end 199.969942 97.78) (width 0.3) (layer "B.Cu") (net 22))
 (segment (start 198.95 71.8) (end 183.6 71.8) (width 0.3) (layer "B.Cu") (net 9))
 (segment (start 167.78 87.62) (end 167.375 87.62) (width 0.3) (layer "B.Cu") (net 9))
 (segment (start 199 71.75) (end 198.95 71.8) (width 0.3) (layer "B.Cu") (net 9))
 (segment (start 183.6 71.8) (end 167.78 87.62) (width 0.3) (layer "B.Cu") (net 9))
 (segment (start 201 83) (end 204.203 86.203) (width 0.3) (layer "B.Cu") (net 18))
 (segment (start 204.203 86.203) (end 204.203 96.362) (width 0.3) (layer "B.Cu") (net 18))
 (segment (start 204.203 96.362) (end 192.625 107.94) (width 0.3) (layer "B.Cu") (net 18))
 (segment (start 203.602 94.997884) (end 195.739884 102.86) (width 0.3) (layer "B.Cu") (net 20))
 (segment (start 201 85.5) (end 203.602 88.102) (width 0.3) (layer "B.Cu") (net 20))
 (segment (start 203.602 88.102) (end 203.602 94.997884) (width 0.3) (layer "B.Cu") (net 20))
 (segment (start 195.739884 102.86) (end 192.625 102.86) (width 0.3) (layer "B.Cu") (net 20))
 (segment (start 199 81.75) (end 197.25 81.75) (width 0.3) (layer "B.Cu") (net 17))
 (segment (start 195.2 83.8) (end 191.515 83.8) (width 0.3) (layer "B.Cu") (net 17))
 (segment (start 191.515 83.8) (end 167.375 107.94) (width 0.3) (layer "B.Cu") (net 17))
 (segment (start 197.25 81.75) (end 195.2 83.8) (width 0.3) (layer "B.Cu") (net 17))
 (segment (start 191.4 91.5) (end 195.1 91.5) (width 0.3) (layer "B.Cu") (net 23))
 (segment (start 190.9 92) (end 191.4 91.5) (width 0.3) (layer "B.Cu") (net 23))
 (segment (start 195.1 91.5) (end 197.35 89.25) (width 0.3) (layer "B.Cu") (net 23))
 (segment (start 190.9 94.1) (end 190.9 92) (width 0.3) (layer "B.Cu") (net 23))
 (segment (start 192.04 95.24) (end 190.9 94.1) (width 0.3) (layer "B.Cu") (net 23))
 (segment (start 192.625 95.24) (end 192.04 95.24) (width 0.3) (layer "B.Cu") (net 23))
 (segment (start 197.35 89.25) (end 199 89.25) (width 0.3) (layer "B.Cu") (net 23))
 (segment (start 199 84.25) (end 196.681 86.569) (width 0.3) (layer "B.Cu") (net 19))
 (segment (start 196.681 86.569) (end 191.789662 86.569) (width 0.3) (layer "B.Cu") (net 19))
 (segment (start 191.789662 86.569) (end 188.898 89.460662) (width 0.3) (layer "B.Cu") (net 19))
 (segment (start 188.898 101.673) (end 192.625 105.4) (width 0.3) (layer "B.Cu") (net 19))
 (segment (start 188.898 89.460662) (end 188.898 101.673) (width 0.3) (layer "B.Cu") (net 19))
 (segment (start 191.535 78.7) (end 198.45 78.7) (width 0.3) (layer "B.Cu") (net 15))
 (segment (start 167.375 102.86) (end 191.535 78.7) (width 0.3) (layer "B.Cu") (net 15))
 (segment (start 198.45 78.7) (end 199 79.25) (width 0.3) (layer "B.Cu") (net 15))
 (segment (start 197.079 88.671) (end 199 86.75) (width 0.3) (layer "B.Cu") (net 21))
 (segment (start 192.625 100.32) (end 189.499 97.194) (width 0.3) (layer "B.Cu") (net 21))
 (segment (start 191.679058 88.671) (end 197.079 88.671) (width 0.3) (layer "B.Cu") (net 21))
 (segment (start 189.499 90.851058) (end 191.679058 88.671) (width 0.3) (layer "B.Cu") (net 21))
 (segment (start 189.499 97.194) (end 189.499 90.851058) (width 0.3) (layer "B.Cu") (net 21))
 (segment (start 146 65.94) (end 147.26 67.2) (width 0.3) (layer "B.Cu") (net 39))
 (segment (start 144.78 65.94) (end 146 65.94) (width 0.3) (layer "B.Cu") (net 39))
 (segment (start 147.3 71) (end 147.26 71.04) (width 0.5) (layer "B.Cu") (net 39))
 (segment (start 147.26 67.2) (end 147.26 71.04) (width 0.3) (layer "B.Cu") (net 39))
 (segment (start 152.34 68.78) (end 152.34 71.04) (width 0.3) (layer "B.Cu") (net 33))
 (segment (start 144.78 63.84) (end 147.4 63.84) (width 0.3) (layer "B.Cu") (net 33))
 (segment (start 147.4 63.84) (end 152.34 68.78) (width 0.3) (layer "B.Cu") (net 33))
 (segment (start 144.84 68.04) (end 144.84 70.92) (width 0.5) (layer "B.Cu") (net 38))
 (segment (start 144.84 70.92) (end 144.72 71.04) (width 0.5) (layer "B.Cu") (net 38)))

